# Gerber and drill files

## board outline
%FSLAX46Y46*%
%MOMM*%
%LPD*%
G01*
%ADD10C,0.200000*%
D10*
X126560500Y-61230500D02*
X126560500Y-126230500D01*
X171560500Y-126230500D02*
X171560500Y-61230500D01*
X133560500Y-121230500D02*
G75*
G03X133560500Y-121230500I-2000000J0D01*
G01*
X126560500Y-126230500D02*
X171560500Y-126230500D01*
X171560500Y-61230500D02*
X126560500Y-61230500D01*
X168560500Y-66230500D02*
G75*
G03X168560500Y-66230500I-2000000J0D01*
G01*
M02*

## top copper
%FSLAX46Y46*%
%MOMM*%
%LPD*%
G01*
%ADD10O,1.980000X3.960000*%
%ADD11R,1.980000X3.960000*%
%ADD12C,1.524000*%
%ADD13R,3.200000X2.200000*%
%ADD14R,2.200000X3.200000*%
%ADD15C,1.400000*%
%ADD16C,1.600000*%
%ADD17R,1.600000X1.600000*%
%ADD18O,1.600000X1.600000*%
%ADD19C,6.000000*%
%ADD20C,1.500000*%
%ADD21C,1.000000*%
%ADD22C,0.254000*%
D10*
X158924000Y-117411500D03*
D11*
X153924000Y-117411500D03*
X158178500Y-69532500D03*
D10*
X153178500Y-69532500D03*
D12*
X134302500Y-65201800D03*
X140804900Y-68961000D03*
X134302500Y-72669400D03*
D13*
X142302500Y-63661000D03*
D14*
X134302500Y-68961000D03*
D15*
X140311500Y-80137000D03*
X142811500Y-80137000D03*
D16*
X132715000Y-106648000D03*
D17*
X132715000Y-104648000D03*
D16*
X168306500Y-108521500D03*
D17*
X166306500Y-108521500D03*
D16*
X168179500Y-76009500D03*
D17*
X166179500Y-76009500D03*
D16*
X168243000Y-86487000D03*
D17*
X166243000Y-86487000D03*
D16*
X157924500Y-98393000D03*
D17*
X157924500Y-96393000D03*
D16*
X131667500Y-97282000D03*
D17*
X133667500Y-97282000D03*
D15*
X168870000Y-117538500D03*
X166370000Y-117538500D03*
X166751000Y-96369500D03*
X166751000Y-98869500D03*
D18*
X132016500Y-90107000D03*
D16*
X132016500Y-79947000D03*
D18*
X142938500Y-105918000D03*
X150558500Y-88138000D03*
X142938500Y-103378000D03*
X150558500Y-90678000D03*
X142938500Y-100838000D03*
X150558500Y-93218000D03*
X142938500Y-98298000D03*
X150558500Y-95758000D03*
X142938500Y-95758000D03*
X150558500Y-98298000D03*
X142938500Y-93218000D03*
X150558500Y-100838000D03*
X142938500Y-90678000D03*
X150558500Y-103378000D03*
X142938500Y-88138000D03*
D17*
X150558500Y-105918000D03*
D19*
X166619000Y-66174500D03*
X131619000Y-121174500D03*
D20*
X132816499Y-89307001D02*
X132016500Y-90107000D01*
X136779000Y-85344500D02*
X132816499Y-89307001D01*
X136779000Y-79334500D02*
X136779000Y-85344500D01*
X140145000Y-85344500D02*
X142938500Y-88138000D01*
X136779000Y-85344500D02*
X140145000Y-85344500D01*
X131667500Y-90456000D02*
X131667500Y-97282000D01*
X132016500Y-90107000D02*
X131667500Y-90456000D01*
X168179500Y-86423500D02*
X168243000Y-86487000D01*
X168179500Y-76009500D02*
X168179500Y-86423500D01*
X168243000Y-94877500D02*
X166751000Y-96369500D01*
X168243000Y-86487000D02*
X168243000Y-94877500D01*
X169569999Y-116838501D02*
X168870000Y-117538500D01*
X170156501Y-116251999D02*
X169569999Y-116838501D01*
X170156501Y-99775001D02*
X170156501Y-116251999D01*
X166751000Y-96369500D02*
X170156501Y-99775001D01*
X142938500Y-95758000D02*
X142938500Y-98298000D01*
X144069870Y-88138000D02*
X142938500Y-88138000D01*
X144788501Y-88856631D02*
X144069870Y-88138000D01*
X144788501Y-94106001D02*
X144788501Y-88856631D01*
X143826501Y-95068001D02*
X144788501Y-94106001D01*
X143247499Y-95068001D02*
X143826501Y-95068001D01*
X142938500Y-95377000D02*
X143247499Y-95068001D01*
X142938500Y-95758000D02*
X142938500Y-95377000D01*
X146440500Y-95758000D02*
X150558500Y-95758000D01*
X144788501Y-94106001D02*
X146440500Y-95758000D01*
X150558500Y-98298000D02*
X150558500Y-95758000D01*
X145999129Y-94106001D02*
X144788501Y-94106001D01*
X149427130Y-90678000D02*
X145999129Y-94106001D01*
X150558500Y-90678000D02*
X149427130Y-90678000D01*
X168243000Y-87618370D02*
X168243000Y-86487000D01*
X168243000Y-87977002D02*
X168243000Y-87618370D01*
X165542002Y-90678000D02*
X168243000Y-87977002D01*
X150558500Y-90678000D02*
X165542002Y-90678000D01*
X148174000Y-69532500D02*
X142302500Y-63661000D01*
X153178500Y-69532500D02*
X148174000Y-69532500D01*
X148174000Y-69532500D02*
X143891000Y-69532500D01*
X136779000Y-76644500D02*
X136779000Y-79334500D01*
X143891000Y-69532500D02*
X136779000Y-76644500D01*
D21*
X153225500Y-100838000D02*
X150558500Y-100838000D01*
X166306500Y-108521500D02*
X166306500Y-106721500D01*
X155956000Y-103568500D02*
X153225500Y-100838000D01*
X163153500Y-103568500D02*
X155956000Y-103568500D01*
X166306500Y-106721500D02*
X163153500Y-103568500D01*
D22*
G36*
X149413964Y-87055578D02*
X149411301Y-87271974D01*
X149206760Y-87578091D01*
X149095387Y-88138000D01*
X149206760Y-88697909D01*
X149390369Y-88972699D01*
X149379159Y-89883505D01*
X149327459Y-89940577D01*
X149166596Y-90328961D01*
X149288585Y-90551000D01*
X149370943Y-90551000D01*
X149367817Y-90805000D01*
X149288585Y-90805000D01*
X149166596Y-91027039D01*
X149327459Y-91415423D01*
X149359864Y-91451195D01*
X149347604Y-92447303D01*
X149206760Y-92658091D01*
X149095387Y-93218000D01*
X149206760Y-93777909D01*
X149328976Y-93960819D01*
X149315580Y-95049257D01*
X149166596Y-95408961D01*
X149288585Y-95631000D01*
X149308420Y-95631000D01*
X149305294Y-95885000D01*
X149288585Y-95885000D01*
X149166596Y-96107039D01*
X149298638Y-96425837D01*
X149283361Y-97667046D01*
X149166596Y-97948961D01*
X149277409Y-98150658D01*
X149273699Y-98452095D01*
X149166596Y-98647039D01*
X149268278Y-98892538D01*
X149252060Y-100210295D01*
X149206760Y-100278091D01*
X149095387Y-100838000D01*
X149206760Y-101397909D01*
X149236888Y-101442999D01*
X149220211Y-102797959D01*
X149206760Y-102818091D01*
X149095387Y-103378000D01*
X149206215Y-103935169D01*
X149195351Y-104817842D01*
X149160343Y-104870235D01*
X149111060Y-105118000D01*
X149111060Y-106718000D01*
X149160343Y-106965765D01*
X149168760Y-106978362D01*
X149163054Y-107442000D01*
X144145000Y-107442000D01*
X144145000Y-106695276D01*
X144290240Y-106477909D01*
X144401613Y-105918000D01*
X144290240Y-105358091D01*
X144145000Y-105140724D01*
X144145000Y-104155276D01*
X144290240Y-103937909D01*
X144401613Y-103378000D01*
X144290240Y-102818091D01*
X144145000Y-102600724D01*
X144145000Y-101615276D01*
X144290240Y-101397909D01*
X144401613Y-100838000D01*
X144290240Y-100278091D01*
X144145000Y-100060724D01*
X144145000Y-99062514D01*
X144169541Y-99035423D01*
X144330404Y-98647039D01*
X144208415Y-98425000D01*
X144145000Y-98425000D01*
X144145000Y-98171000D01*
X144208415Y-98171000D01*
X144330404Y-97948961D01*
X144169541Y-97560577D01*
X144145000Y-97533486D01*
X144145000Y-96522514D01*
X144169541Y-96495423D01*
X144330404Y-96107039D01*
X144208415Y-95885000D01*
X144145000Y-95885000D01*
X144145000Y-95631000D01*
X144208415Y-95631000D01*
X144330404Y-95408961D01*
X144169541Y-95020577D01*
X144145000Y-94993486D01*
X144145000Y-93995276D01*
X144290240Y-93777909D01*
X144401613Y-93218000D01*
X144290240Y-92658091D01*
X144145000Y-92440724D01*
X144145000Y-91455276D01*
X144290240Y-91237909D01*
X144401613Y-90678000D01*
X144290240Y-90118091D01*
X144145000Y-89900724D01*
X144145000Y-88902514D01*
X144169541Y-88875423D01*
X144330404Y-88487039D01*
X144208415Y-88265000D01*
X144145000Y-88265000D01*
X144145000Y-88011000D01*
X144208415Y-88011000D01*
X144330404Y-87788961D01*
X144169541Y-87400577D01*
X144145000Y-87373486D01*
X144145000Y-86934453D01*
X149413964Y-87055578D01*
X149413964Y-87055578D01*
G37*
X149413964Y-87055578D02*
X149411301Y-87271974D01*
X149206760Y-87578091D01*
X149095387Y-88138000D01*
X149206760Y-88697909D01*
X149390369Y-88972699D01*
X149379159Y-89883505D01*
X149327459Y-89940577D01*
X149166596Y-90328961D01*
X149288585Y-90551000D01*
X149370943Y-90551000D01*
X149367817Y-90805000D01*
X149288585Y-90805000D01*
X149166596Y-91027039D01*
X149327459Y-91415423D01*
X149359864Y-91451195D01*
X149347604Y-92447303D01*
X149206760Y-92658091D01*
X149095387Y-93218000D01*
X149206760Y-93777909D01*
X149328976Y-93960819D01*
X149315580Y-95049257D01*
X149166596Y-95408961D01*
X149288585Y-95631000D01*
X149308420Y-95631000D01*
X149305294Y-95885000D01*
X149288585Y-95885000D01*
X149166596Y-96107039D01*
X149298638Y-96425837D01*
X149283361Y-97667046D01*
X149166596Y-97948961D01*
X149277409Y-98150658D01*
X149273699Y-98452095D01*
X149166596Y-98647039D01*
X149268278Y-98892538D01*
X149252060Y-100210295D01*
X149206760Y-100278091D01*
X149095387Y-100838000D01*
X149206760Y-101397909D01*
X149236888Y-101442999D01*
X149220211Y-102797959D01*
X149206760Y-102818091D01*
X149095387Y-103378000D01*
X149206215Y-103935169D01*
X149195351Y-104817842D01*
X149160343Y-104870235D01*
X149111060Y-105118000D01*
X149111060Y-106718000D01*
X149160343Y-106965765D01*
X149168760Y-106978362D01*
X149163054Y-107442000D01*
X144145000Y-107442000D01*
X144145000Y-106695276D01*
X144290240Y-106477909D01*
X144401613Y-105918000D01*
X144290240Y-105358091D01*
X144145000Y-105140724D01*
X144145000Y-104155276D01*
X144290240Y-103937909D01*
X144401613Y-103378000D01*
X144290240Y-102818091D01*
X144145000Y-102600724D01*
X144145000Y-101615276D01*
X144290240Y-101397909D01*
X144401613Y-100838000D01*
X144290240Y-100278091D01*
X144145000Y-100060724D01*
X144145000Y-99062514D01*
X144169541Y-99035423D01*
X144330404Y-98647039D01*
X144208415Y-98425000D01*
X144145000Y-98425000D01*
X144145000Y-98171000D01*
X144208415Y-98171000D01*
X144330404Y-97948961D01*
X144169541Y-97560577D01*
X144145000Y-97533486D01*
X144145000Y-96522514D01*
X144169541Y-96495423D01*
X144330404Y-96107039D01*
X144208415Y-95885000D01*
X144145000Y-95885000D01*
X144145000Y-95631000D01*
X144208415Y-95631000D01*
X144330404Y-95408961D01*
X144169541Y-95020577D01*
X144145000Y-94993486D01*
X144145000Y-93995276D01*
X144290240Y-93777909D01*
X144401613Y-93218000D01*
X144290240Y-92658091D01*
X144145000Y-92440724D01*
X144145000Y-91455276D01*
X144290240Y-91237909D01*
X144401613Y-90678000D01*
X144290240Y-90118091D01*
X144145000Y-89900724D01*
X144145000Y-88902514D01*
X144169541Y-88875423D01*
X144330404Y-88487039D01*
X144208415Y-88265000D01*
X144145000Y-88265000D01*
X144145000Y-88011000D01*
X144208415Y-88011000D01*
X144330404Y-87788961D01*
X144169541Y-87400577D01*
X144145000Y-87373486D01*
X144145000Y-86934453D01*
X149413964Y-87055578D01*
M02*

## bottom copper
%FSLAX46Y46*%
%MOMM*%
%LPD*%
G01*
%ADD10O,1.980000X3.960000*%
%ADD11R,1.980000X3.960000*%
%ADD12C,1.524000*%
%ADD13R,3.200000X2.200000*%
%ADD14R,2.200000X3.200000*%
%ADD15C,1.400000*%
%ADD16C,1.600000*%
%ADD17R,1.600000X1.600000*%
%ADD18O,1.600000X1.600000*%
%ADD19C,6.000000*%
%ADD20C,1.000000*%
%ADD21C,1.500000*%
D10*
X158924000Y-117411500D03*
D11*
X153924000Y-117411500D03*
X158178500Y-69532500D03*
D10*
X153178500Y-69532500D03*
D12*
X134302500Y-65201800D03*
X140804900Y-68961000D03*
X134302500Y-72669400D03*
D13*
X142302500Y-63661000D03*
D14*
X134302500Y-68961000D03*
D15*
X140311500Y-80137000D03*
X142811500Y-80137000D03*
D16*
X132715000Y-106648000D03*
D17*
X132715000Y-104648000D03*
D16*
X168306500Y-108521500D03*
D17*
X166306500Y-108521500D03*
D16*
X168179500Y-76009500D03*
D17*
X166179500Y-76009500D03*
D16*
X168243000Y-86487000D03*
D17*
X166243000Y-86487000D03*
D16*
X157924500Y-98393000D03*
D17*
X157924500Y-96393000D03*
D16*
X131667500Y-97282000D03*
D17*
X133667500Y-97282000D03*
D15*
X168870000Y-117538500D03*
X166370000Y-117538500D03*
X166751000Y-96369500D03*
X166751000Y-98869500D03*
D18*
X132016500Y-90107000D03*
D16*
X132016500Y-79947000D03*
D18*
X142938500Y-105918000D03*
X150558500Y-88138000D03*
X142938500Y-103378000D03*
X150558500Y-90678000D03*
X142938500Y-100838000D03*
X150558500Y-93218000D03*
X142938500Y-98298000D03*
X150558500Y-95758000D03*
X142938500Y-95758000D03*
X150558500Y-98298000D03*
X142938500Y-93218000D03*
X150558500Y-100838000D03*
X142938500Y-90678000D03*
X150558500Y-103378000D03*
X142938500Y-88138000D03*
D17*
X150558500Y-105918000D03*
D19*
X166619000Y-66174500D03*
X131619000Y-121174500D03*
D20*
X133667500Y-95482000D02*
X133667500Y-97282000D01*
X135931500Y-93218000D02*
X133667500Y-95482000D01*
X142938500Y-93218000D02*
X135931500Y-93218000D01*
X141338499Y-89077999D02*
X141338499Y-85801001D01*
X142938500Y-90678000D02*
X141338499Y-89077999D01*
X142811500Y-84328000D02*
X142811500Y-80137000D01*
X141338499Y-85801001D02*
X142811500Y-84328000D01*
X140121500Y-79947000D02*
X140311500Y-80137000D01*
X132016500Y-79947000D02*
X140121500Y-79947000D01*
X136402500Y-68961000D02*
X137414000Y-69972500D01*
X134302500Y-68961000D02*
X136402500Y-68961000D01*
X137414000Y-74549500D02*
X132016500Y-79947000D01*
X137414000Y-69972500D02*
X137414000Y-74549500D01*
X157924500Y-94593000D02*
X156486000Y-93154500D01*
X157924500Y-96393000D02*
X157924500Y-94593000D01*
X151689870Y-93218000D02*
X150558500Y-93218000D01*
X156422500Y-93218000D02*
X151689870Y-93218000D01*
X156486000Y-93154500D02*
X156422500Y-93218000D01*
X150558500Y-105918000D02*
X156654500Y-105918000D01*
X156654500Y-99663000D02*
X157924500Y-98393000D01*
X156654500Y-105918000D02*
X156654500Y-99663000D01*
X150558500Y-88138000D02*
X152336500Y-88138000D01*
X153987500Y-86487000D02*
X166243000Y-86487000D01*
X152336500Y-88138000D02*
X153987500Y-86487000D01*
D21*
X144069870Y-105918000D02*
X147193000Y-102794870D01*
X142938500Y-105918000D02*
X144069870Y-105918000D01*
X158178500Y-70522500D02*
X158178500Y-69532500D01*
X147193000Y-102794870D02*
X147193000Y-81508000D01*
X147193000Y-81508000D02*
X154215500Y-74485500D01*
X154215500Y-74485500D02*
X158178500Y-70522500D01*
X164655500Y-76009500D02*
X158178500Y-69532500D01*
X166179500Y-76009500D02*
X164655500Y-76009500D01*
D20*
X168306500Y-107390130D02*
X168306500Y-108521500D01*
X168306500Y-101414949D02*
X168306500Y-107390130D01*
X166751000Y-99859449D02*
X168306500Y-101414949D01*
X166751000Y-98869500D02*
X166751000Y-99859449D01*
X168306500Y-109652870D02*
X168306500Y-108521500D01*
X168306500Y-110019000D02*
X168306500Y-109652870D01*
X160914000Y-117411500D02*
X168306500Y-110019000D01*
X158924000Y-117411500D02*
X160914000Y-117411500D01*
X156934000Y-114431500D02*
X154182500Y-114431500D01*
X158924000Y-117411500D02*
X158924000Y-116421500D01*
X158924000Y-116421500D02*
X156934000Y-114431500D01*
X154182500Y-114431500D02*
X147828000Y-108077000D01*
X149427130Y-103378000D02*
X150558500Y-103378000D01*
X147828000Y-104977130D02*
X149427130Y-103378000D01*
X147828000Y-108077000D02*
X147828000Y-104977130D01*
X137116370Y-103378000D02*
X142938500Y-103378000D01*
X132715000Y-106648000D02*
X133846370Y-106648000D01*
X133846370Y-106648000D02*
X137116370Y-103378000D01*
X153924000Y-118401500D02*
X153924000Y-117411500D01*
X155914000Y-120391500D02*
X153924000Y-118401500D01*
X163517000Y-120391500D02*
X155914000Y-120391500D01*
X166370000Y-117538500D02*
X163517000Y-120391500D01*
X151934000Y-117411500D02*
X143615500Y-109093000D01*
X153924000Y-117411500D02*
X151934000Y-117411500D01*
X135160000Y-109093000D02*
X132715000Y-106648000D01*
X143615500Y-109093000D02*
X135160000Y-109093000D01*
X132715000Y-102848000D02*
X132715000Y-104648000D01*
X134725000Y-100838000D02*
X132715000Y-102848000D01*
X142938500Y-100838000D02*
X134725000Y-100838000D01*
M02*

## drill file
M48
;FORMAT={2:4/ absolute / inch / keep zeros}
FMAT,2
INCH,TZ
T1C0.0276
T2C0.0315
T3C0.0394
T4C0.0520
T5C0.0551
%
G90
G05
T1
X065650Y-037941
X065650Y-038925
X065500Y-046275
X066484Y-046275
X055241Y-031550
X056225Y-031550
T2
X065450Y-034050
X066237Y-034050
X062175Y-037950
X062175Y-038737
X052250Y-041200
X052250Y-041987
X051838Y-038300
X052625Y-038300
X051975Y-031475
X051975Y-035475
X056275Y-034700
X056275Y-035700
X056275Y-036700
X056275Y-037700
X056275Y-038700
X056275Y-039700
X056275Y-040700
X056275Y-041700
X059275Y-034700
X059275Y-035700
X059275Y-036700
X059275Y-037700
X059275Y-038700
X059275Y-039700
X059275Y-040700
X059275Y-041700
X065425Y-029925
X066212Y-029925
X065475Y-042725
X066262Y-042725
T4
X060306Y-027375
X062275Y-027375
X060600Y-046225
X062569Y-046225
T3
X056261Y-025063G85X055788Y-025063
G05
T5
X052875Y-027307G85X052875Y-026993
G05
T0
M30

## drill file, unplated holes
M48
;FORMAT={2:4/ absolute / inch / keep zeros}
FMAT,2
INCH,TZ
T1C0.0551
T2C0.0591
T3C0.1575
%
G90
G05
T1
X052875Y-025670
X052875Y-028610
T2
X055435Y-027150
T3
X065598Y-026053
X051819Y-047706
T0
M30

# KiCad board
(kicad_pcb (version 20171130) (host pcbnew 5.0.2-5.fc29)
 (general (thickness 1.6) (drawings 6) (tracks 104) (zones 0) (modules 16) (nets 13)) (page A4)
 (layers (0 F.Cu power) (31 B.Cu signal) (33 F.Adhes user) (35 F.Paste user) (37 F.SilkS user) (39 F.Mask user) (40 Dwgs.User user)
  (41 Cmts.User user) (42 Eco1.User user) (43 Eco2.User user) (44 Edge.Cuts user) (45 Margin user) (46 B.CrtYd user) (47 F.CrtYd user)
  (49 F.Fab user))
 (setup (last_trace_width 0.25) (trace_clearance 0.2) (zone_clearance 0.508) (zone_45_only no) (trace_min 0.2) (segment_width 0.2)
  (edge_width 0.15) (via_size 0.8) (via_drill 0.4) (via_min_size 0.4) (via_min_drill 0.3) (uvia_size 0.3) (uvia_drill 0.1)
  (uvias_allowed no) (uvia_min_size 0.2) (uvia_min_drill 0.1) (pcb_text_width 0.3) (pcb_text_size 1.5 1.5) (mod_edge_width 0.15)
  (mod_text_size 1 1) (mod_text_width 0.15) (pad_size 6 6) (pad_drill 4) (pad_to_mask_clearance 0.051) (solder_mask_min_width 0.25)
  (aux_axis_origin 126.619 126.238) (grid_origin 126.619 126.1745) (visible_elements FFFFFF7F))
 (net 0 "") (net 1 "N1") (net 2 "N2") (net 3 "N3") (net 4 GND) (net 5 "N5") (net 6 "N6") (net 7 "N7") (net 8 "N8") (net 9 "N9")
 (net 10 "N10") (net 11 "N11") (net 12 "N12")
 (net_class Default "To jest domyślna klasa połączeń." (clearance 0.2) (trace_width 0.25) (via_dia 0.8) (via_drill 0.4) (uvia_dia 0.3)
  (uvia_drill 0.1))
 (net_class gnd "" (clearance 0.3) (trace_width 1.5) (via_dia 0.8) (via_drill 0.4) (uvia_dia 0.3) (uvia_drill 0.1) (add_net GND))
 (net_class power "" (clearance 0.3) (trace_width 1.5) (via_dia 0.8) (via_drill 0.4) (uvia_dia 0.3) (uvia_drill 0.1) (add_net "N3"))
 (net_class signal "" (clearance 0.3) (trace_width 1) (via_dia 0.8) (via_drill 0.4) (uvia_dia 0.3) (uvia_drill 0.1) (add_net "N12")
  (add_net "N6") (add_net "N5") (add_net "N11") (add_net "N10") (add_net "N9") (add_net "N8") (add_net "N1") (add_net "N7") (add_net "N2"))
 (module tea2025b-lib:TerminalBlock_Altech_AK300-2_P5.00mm (layer F.Cu) (at 153.924 117.4115)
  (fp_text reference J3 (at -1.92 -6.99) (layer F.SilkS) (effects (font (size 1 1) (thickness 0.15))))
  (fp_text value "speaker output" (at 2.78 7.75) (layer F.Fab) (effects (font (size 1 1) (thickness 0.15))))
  (pad 2 thru_hole oval (at 5 0) (size 1.98 3.96) (drill 1.32) (layers *.Cu *.Mask) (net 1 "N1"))
  (pad 1 thru_hole rect (at 0 0) (size 1.98 3.96) (drill 1.32) (layers *.Cu *.Mask) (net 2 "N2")))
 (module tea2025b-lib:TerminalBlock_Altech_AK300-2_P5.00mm (layer F.Cu) (at 158.1785 69.5325 180)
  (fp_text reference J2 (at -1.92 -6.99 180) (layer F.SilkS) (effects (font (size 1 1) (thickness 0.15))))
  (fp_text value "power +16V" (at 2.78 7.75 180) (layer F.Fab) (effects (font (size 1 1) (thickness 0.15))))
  (pad 1 thru_hole rect (at 0 0 180) (size 1.98 3.96) (drill 1.32) (layers *.Cu *.Mask) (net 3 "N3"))
  (pad 2 thru_hole oval (at 5 0 180) (size 1.98 3.96) (drill 1.32) (layers *.Cu *.Mask) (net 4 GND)))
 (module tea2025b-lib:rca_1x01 (layer F.Cu) (at 134.3025 68.961 90)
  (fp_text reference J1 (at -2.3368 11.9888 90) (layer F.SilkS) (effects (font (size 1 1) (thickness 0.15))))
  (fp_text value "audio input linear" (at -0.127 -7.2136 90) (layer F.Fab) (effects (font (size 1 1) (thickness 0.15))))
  (pad 1 thru_hole rect (at 0 0 90) (size 3.2 2.2) (drill oval 2.2 1.4) (layers *.Cu *.Mask) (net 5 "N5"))
  (pad 2 thru_hole rect (at 5.3 8 180) (size 3.2 2.2) (drill oval 2.2 1) (layers *.Cu *.Mask) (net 4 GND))
  (pad "" np_thru_hole circle (at -3.7084 0 90) (size 1.524 1.524) (drill 1.4) (layers *.Cu *.Mask))
  (pad "" np_thru_hole circle (at 0 6.5024 90) (size 1.524 1.524) (drill 1.5) (layers *.Cu *.Mask))
  (pad "" np_thru_hole circle (at 3.7592 0 90) (size 1.524 1.524) (drill 1.4) (layers *.Cu *.Mask)))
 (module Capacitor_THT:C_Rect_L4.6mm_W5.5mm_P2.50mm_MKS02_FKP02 (layer F.Cu) (at 142.8115 80.137 180)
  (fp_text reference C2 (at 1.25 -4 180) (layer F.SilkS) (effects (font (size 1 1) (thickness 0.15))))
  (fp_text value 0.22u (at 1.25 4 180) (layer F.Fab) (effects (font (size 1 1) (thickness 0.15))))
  (pad 2 thru_hole circle (at 2.5 0 180) (size 1.4 1.4) (drill 0.7) (layers *.Cu *.Mask) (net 5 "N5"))
  (pad 1 thru_hole circle (at 0 0 180) (size 1.4 1.4) (drill 0.7) (layers *.Cu *.Mask) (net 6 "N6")))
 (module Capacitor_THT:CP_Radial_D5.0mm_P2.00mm (layer F.Cu) (at 132.715 104.648 270)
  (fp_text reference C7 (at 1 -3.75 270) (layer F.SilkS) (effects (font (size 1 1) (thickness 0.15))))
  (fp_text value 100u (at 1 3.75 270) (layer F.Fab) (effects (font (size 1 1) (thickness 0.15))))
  (pad 2 thru_hole circle (at 2 0 270) (size 1.6 1.6) (drill 0.8) (layers *.Cu *.Mask) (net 2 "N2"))
  (pad 1 thru_hole rect (at 0 0 270) (size 1.6 1.6) (drill 0.8) (layers *.Cu *.Mask) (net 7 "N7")))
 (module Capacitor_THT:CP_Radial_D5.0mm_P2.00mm (layer F.Cu) (at 166.3065 108.5215)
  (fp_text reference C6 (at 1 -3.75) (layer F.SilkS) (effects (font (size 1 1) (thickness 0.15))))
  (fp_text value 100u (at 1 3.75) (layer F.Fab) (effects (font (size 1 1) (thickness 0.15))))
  (pad 2 thru_hole circle (at 2 0) (size 1.6 1.6) (drill 0.8) (layers *.Cu *.Mask) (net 1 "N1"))
  (pad 1 thru_hole rect (at 0 0) (size 1.6 1.6) (drill 0.8) (layers *.Cu *.Mask) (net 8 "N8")))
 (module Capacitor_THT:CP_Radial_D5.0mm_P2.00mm (layer F.Cu) (at 166.1795 76.0095)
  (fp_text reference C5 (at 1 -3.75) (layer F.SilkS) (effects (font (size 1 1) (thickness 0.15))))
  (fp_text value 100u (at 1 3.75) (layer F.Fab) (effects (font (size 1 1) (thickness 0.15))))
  (pad 2 thru_hole circle (at 2 0) (size 1.6 1.6) (drill 0.8) (layers *.Cu *.Mask) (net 4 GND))
  (pad 1 thru_hole rect (at 0 0) (size 1.6 1.6) (drill 0.8) (layers *.Cu *.Mask) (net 3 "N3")))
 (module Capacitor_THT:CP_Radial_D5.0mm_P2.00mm (layer F.Cu) (at 166.243 86.487)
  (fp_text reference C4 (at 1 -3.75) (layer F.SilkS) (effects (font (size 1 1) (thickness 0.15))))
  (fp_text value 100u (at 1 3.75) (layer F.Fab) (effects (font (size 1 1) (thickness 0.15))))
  (pad 2 thru_hole circle (at 2 0) (size 1.6 1.6) (drill 0.8) (layers *.Cu *.Mask) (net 4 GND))
  (pad 1 thru_hole rect (at 0 0) (size 1.6 1.6) (drill 0.8) (layers *.Cu *.Mask) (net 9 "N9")))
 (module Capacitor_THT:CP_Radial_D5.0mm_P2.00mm (layer F.Cu) (at 157.9245 96.393 270)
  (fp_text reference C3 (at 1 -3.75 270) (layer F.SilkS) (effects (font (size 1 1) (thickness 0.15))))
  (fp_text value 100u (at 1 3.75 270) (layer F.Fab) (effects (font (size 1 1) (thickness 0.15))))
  (pad 2 thru_hole circle (at 2 0 270) (size 1.6 1.6) (drill 0.8) (layers *.Cu *.Mask) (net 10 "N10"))
  (pad 1 thru_hole rect (at 0 0 270) (size 1.6 1.6) (drill 0.8) (layers *.Cu *.Mask) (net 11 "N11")))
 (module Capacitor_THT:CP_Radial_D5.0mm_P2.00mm (layer F.Cu) (at 133.6675 97.282 180)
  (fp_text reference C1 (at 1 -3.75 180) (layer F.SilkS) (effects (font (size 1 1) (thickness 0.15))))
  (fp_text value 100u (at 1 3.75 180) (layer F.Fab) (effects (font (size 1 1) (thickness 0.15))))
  (pad 2 thru_hole circle (at 2 0 180) (size 1.6 1.6) (drill 0.8) (layers *.Cu *.Mask) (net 4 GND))
  (pad 1 thru_hole rect (at 0 0 180) (size 1.6 1.6) (drill 0.8) (layers *.Cu *.Mask) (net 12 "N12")))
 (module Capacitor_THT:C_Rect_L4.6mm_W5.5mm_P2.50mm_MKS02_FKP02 (layer F.Cu) (at 166.37 117.5385)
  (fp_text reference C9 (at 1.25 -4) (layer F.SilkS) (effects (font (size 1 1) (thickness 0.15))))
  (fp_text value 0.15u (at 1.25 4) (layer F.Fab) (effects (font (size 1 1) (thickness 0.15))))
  (pad 2 thru_hole circle (at 2.5 0) (size 1.4 1.4) (drill 0.7) (layers *.Cu *.Mask) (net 4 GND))
  (pad 1 thru_hole circle (at 0 0) (size 1.4 1.4) (drill 0.7) (layers *.Cu *.Mask) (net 2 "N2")))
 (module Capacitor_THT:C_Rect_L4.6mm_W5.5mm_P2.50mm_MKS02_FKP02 (layer F.Cu) (at 166.751 98.8695 90)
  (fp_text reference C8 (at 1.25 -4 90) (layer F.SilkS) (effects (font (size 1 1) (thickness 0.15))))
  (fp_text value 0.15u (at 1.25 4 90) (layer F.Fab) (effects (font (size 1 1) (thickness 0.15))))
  (pad 2 thru_hole circle (at 2.5 0 90) (size 1.4 1.4) (drill 0.7) (layers *.Cu *.Mask) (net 4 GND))
  (pad 1 thru_hole circle (at 0 0 90) (size 1.4 1.4) (drill 0.7) (layers *.Cu *.Mask) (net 1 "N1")))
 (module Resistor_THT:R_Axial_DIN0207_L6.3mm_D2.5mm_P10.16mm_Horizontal (layer F.Cu) (at 132.0165 79.947 270)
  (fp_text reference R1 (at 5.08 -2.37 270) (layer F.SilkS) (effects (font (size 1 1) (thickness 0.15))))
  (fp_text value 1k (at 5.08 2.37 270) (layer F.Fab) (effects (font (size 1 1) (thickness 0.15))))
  (pad 2 thru_hole oval (at 10.16 0 270) (size 1.6 1.6) (drill 0.8) (layers *.Cu *.Mask) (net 4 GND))
  (pad 1 thru_hole circle (at 0 0 270) (size 1.6 1.6) (drill 0.8) (layers *.Cu *.Mask) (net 5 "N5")))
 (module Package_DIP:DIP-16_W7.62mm (layer F.Cu) (at 150.5585 105.918 180)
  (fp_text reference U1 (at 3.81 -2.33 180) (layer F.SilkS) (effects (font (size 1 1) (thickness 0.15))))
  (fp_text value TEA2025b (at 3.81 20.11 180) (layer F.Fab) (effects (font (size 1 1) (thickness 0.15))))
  (pad 16 thru_hole oval (at 7.62 0 180) (size 1.6 1.6) (drill 0.8) (layers *.Cu *.Mask) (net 3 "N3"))
  (pad 8 thru_hole oval (at 0 17.78 180) (size 1.6 1.6) (drill 0.8) (layers *.Cu *.Mask) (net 9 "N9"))
  (pad 15 thru_hole oval (at 7.62 2.54 180) (size 1.6 1.6) (drill 0.8) (layers *.Cu *.Mask) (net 2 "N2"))
  (pad 7 thru_hole oval (at 0 15.24 180) (size 1.6 1.6) (drill 0.8) (layers *.Cu *.Mask) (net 4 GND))
  (pad 14 thru_hole oval (at 7.62 5.08 180) (size 1.6 1.6) (drill 0.8) (layers *.Cu *.Mask) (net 7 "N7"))
  (pad 6 thru_hole oval (at 0 12.7 180) (size 1.6 1.6) (drill 0.8) (layers *.Cu *.Mask) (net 11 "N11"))
  (pad 13 thru_hole oval (at 7.62 7.62 180) (size 1.6 1.6) (drill 0.8) (layers *.Cu *.Mask) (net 4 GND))
  (pad 5 thru_hole oval (at 0 10.16 180) (size 1.6 1.6) (drill 0.8) (layers *.Cu *.Mask) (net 4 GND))
  (pad 12 thru_hole oval (at 7.62 10.16 180) (size 1.6 1.6) (drill 0.8) (layers *.Cu *.Mask) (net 4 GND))
  (pad 4 thru_hole oval (at 0 7.62 180) (size 1.6 1.6) (drill 0.8) (layers *.Cu *.Mask) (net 4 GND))
  (pad 11 thru_hole oval (at 7.62 12.7 180) (size 1.6 1.6) (drill 0.8) (layers *.Cu *.Mask) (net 12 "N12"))
  (pad 3 thru_hole oval (at 0 5.08 180) (size 1.6 1.6) (drill 0.8) (layers *.Cu *.Mask) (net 8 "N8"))
  (pad 10 thru_hole oval (at 7.62 15.24 180) (size 1.6 1.6) (drill 0.8) (layers *.Cu *.Mask) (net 6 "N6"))
  (pad 2 thru_hole oval (at 0 2.54 180) (size 1.6 1.6) (drill 0.8) (layers *.Cu *.Mask) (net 1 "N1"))
  (pad 9 thru_hole oval (at 7.62 17.78 180) (size 1.6 1.6) (drill 0.8) (layers *.Cu *.Mask) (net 4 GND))
  (pad 1 thru_hole rect (at 0 0 180) (size 1.6 1.6) (drill 0.8) (layers *.Cu *.Mask) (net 10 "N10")))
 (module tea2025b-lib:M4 (layer F.Cu) (at 166.619 66.1745)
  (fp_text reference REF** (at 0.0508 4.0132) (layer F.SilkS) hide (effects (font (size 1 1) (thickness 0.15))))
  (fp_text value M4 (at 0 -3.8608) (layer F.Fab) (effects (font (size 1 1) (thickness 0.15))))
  (pad "" np_thru_hole circle (at 0 0) (size 6 6) (drill 4) (layers *.Cu *.Mask)))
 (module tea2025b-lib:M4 (layer F.Cu) (at 131.619 121.1745)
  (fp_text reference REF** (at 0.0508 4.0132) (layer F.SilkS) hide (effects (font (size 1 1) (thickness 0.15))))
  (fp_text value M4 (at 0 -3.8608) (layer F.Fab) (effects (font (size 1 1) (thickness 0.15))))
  (pad "" np_thru_hole circle (at 0 0) (size 6 6) (drill 4) (layers *.Cu *.Mask)))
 (gr_line (start 126.5605 61.2305) (end 126.5605 126.2305) (layer Edge.Cuts) (width 0.2))
 (gr_line (start 171.5605 126.2305) (end 171.5605 61.2305) (layer Edge.Cuts) (width 0.2))
 (gr_circle (center 131.5605 121.2305) (end 133.5605 121.2305) (layer Edge.Cuts) (width 0.2))
 (gr_line (start 126.5605 126.2305) (end 171.5605 126.2305) (layer Edge.Cuts) (width 0.2))
 (gr_line (start 171.5605 61.2305) (end 126.5605 61.2305) (layer Edge.Cuts) (width 0.2))
 (gr_circle (center 166.5605 66.2305) (end 168.5605 66.2305) (layer Edge.Cuts) (width 0.2))
 (segment (start 132.816499 89.307001) (end 132.0165 90.107) (width 1.5) (layer F.Cu) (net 4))
 (segment (start 136.779 85.3445) (end 132.816499 89.307001) (width 1.5) (layer F.Cu) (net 4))
 (segment (start 136.779 79.3345) (end 136.779 85.3445) (width 1.5) (layer F.Cu) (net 4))
 (segment (start 140.145 85.3445) (end 142.9385 88.138) (width 1.5) (layer F.Cu) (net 4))
 (segment (start 136.779 85.3445) (end 140.145 85.3445) (width 1.5) (layer F.Cu) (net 4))
 (segment (start 131.6675 90.456) (end 131.6675 97.282) (width 1.5) (layer F.Cu) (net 4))
 (segment (start 132.0165 90.107) (end 131.6675 90.456) (width 1.5) (layer F.Cu) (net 4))
 (segment (start 168.1795 86.4235) (end 168.243 86.487) (width 1.5) (layer F.Cu) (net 4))
 (segment (start 168.1795 76.0095) (end 168.1795 86.4235) (width 1.5) (layer F.Cu) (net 4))
 (segment (start 168.243 94.8775) (end 166.751 96.3695) (width 1.5) (layer F.Cu) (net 4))
 (segment (start 168.243 86.487) (end 168.243 94.8775) (width 1.5) (layer F.Cu) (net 4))
 (segment (start 169.569999 116.838501) (end 168.87 117.5385) (width 1.5) (layer F.Cu) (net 4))
 (segment (start 170.156501 116.251999) (end 169.569999 116.838501) (width 1.5) (layer F.Cu) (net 4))
 (segment (start 170.156501 99.775001) (end 170.156501 116.251999) (width 1.5) (layer F.Cu) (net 4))
 (segment (start 166.751 96.3695) (end 170.156501 99.775001) (width 1.5) (layer F.Cu) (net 4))
 (segment (start 142.9385 95.758) (end 142.9385 98.298) (width 1.5) (layer F.Cu) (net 4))
 (segment (start 144.06987 88.138) (end 142.9385 88.138) (width 1.5) (layer F.Cu) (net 4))
 (segment (start 144.788501 88.856631) (end 144.06987 88.138) (width 1.5) (layer F.Cu) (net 4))
 (segment (start 144.788501 94.106001) (end 144.788501 88.856631) (width 1.5) (layer F.Cu) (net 4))
 (segment (start 143.826501 95.068001) (end 144.788501 94.106001) (width 1.5) (layer F.Cu) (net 4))
 (segment (start 143.247499 95.068001) (end 143.826501 95.068001) (width 1.5) (layer F.Cu) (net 4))
 (segment (start 142.9385 95.377) (end 143.247499 95.068001) (width 1.5) (layer F.Cu) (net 4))
 (segment (start 142.9385 95.758) (end 142.9385 95.377) (width 1.5) (layer F.Cu) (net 4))
 (segment (start 146.4405 95.758) (end 150.5585 95.758) (width 1.5) (layer F.Cu) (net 4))
 (segment (start 144.788501 94.106001) (end 146.4405 95.758) (width 1.5) (layer F.Cu) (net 4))
 (segment (start 150.5585 98.298) (end 150.5585 95.758) (width 1.5) (layer F.Cu) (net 4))
 (segment (start 145.999129 94.106001) (end 144.788501 94.106001) (width 1.5) (layer F.Cu) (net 4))
 (segment (start 149.42713 90.678) (end 145.999129 94.106001) (width 1.5) (layer F.Cu) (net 4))
 (segment (start 150.5585 90.678) (end 149.42713 90.678) (width 1.5) (layer F.Cu) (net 4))
 (segment (start 168.243 87.61837) (end 168.243 86.487) (width 1.5) (layer F.Cu) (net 4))
 (segment (start 168.243 87.977002) (end 168.243 87.61837) (width 1.5) (layer F.Cu) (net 4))
 (segment (start 165.542002 90.678) (end 168.243 87.977002) (width 1.5) (layer F.Cu) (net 4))
 (segment (start 150.5585 90.678) (end 165.542002 90.678) (width 1.5) (layer F.Cu) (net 4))
 (segment (start 148.174 69.5325) (end 142.3025 63.661) (width 1.5) (layer F.Cu) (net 4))
 (segment (start 153.1785 69.5325) (end 148.174 69.5325) (width 1.5) (layer F.Cu) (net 4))
 (segment (start 148.174 69.5325) (end 143.891 69.5325) (width 1.5) (layer F.Cu) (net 4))
 (segment (start 136.779 76.6445) (end 136.779 79.3345) (width 1.5) (layer F.Cu) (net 4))
 (segment (start 143.891 69.5325) (end 136.779 76.6445) (width 1.5) (layer F.Cu) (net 4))
 (segment (start 133.6675 95.482) (end 133.6675 97.282) (width 1) (layer B.Cu) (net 12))
 (segment (start 135.9315 93.218) (end 133.6675 95.482) (width 1) (layer B.Cu) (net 12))
 (segment (start 142.9385 93.218) (end 135.9315 93.218) (width 1) (layer B.Cu) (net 12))
 (segment (start 141.338499 89.077999) (end 141.338499 85.801001) (width 1) (layer B.Cu) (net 6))
 (segment (start 142.9385 90.678) (end 141.338499 89.077999) (width 1) (layer B.Cu) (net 6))
 (segment (start 142.8115 84.328) (end 142.8115 80.137) (width 1) (layer B.Cu) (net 6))
 (segment (start 141.338499 85.801001) (end 142.8115 84.328) (width 1) (layer B.Cu) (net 6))
 (segment (start 140.1215 79.947) (end 140.3115 80.137) (width 1) (layer B.Cu) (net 5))
 (segment (start 132.0165 79.947) (end 140.1215 79.947) (width 1) (layer B.Cu) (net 5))
 (segment (start 136.4025 68.961) (end 137.414 69.9725) (width 1) (layer B.Cu) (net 5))
 (segment (start 134.3025 68.961) (end 136.4025 68.961) (width 1) (layer B.Cu) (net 5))
 (segment (start 137.414 74.5495) (end 132.0165 79.947) (width 1) (layer B.Cu) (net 5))
 (segment (start 137.414 69.9725) (end 137.414 74.5495) (width 1) (layer B.Cu) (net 5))
 (segment (start 157.9245 94.593) (end 156.486 93.1545) (width 1) (layer B.Cu) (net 11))
 (segment (start 157.9245 96.393) (end 157.9245 94.593) (width 1) (layer B.Cu) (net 11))
 (segment (start 151.68987 93.218) (end 150.5585 93.218) (width 1) (layer B.Cu) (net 11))
 (segment (start 156.4225 93.218) (end 151.68987 93.218) (width 1) (layer B.Cu) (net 11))
 (segment (start 156.486 93.1545) (end 156.4225 93.218) (width 1) (layer B.Cu) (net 11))
 (segment (start 150.5585 105.918) (end 156.6545 105.918) (width 1) (layer B.Cu) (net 10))
 (segment (start 156.6545 99.663) (end 157.9245 98.393) (width 1) (layer B.Cu) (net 10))
 (segment (start 156.6545 105.918) (end 156.6545 99.663) (width 1) (layer B.Cu) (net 10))
 (segment (start 150.5585 88.138) (end 152.3365 88.138) (width 1) (layer B.Cu) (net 9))
 (segment (start 153.9875 86.487) (end 166.243 86.487) (width 1) (layer B.Cu) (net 9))
 (segment (start 152.3365 88.138) (end 153.9875 86.487) (width 1) (layer B.Cu) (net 9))
 (segment (start 144.06987 105.918) (end 147.193 102.79487) (width 1.5) (layer B.Cu) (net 3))
 (segment (start 142.9385 105.918) (end 144.06987 105.918) (width 1.5) (layer B.Cu) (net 3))
 (segment (start 158.1785 70.5225) (end 158.1785 69.5325) (width 1.5) (layer B.Cu) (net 3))
 (segment (start 147.193 102.79487) (end 147.193 81.508) (width 1.5) (layer B.Cu) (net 3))
 (segment (start 147.193 81.508) (end 154.2155 74.4855) (width 1.5) (layer B.Cu) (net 3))
 (segment (start 154.2155 74.4855) (end 158.1785 70.5225) (width 1.5) (layer B.Cu) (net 3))
 (segment (start 164.6555 76.0095) (end 158.1785 69.5325) (width 1.5) (layer B.Cu) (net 3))
 (segment (start 166.1795 76.0095) (end 164.6555 76.0095) (width 1.5) (layer B.Cu) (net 3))
 (segment (start 168.3065 107.39013) (end 168.3065 108.5215) (width 1) (layer B.Cu) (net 1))
 (segment (start 168.3065 101.414949) (end 168.3065 107.39013) (width 1) (layer B.Cu) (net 1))
 (segment (start 166.751 99.859449) (end 168.3065 101.414949) (width 1) (layer B.Cu) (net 1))
 (segment (start 166.751 98.8695) (end 166.751 99.859449) (width 1) (layer B.Cu) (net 1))
 (segment (start 168.3065 109.65287) (end 168.3065 108.5215) (width 1) (layer B.Cu) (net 1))
 (segment (start 168.3065 110.019) (end 168.3065 109.65287) (width 1) (layer B.Cu) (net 1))
 (segment (start 160.914 117.4115) (end 168.3065 110.019) (width 1) (layer B.Cu) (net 1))
 (segment (start 158.924 117.4115) (end 160.914 117.4115) (width 1) (layer B.Cu) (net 1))
 (segment (start 156.934 114.4315) (end 154.1825 114.4315) (width 1) (layer B.Cu) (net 1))
 (segment (start 158.924 117.4115) (end 158.924 116.4215) (width 1) (layer B.Cu) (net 1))
 (segment (start 158.924 116.4215) (end 156.934 114.4315) (width 1) (layer B.Cu) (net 1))
 (segment (start 154.1825 114.4315) (end 147.828 108.077) (width 1) (layer B.Cu) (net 1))
 (segment (start 149.42713 103.378) (end 150.5585 103.378) (width 1) (layer B.Cu) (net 1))
 (segment (start 147.828 104.97713) (end 149.42713 103.378) (width 1) (layer B.Cu) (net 1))
 (segment (start 147.828 108.077) (end 147.828 104.97713) (width 1) (layer B.Cu) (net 1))
 (segment (start 153.2255 100.838) (end 150.5585 100.838) (width 1) (layer F.Cu) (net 8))
 (segment (start 166.3065 108.5215) (end 166.3065 106.7215) (width 1) (layer F.Cu) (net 8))
 (segment (start 155.956 103.5685) (end 153.2255 100.838) (width 1) (layer F.Cu) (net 8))
 (segment (start 163.1535 103.5685) (end 155.956 103.5685) (width 1) (layer F.Cu) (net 8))
 (segment (start 166.3065 106.7215) (end 163.1535 103.5685) (width 1) (layer F.Cu) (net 8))
 (segment (start 137.11637 103.378) (end 142.9385 103.378) (width 1) (layer B.Cu) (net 2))
 (segment (start 132.715 106.648) (end 133.84637 106.648) (width 1) (layer B.Cu) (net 2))
 (segment (start 133.84637 106.648) (end 137.11637 103.378) (width 1) (layer B.Cu) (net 2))
 (segment (start 153.924 118.4015) (end 153.924 117.4115) (width 1) (layer B.Cu) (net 2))
 (segment (start 155.914 120.3915) (end 153.924 118.4015) (width 1) (layer B.Cu) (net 2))
 (segment (start 163.517 120.3915) (end 155.914 120.3915) (width 1) (layer B.Cu) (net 2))
 (segment (start 166.37 117.5385) (end 163.517 120.3915) (width 1) (layer B.Cu) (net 2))
 (segment (start 151.934 117.4115) (end 143.6155 109.093) (width 1) (layer B.Cu) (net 2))
 (segment (start 153.924 117.4115) (end 151.934 117.4115) (width 1) (layer B.Cu) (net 2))
 (segment (start 135.16 109.093) (end 132.715 106.648) (width 1) (layer B.Cu) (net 2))
 (segment (start 143.6155 109.093) (end 135.16 109.093) (width 1) (layer B.Cu) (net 2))
 (segment (start 132.715 102.848) (end 132.715 104.648) (width 1) (layer B.Cu) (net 7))
 (segment (start 134.725 100.838) (end 132.715 102.848) (width 1) (layer B.Cu) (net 7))
 (segment (start 142.9385 100.838) (end 134.725 100.838) (width 1) (layer B.Cu) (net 7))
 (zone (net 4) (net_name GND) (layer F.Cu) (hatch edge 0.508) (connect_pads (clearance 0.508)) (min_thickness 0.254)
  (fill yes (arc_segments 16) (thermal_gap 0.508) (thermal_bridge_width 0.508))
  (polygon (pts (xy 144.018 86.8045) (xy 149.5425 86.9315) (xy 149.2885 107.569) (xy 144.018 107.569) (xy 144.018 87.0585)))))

